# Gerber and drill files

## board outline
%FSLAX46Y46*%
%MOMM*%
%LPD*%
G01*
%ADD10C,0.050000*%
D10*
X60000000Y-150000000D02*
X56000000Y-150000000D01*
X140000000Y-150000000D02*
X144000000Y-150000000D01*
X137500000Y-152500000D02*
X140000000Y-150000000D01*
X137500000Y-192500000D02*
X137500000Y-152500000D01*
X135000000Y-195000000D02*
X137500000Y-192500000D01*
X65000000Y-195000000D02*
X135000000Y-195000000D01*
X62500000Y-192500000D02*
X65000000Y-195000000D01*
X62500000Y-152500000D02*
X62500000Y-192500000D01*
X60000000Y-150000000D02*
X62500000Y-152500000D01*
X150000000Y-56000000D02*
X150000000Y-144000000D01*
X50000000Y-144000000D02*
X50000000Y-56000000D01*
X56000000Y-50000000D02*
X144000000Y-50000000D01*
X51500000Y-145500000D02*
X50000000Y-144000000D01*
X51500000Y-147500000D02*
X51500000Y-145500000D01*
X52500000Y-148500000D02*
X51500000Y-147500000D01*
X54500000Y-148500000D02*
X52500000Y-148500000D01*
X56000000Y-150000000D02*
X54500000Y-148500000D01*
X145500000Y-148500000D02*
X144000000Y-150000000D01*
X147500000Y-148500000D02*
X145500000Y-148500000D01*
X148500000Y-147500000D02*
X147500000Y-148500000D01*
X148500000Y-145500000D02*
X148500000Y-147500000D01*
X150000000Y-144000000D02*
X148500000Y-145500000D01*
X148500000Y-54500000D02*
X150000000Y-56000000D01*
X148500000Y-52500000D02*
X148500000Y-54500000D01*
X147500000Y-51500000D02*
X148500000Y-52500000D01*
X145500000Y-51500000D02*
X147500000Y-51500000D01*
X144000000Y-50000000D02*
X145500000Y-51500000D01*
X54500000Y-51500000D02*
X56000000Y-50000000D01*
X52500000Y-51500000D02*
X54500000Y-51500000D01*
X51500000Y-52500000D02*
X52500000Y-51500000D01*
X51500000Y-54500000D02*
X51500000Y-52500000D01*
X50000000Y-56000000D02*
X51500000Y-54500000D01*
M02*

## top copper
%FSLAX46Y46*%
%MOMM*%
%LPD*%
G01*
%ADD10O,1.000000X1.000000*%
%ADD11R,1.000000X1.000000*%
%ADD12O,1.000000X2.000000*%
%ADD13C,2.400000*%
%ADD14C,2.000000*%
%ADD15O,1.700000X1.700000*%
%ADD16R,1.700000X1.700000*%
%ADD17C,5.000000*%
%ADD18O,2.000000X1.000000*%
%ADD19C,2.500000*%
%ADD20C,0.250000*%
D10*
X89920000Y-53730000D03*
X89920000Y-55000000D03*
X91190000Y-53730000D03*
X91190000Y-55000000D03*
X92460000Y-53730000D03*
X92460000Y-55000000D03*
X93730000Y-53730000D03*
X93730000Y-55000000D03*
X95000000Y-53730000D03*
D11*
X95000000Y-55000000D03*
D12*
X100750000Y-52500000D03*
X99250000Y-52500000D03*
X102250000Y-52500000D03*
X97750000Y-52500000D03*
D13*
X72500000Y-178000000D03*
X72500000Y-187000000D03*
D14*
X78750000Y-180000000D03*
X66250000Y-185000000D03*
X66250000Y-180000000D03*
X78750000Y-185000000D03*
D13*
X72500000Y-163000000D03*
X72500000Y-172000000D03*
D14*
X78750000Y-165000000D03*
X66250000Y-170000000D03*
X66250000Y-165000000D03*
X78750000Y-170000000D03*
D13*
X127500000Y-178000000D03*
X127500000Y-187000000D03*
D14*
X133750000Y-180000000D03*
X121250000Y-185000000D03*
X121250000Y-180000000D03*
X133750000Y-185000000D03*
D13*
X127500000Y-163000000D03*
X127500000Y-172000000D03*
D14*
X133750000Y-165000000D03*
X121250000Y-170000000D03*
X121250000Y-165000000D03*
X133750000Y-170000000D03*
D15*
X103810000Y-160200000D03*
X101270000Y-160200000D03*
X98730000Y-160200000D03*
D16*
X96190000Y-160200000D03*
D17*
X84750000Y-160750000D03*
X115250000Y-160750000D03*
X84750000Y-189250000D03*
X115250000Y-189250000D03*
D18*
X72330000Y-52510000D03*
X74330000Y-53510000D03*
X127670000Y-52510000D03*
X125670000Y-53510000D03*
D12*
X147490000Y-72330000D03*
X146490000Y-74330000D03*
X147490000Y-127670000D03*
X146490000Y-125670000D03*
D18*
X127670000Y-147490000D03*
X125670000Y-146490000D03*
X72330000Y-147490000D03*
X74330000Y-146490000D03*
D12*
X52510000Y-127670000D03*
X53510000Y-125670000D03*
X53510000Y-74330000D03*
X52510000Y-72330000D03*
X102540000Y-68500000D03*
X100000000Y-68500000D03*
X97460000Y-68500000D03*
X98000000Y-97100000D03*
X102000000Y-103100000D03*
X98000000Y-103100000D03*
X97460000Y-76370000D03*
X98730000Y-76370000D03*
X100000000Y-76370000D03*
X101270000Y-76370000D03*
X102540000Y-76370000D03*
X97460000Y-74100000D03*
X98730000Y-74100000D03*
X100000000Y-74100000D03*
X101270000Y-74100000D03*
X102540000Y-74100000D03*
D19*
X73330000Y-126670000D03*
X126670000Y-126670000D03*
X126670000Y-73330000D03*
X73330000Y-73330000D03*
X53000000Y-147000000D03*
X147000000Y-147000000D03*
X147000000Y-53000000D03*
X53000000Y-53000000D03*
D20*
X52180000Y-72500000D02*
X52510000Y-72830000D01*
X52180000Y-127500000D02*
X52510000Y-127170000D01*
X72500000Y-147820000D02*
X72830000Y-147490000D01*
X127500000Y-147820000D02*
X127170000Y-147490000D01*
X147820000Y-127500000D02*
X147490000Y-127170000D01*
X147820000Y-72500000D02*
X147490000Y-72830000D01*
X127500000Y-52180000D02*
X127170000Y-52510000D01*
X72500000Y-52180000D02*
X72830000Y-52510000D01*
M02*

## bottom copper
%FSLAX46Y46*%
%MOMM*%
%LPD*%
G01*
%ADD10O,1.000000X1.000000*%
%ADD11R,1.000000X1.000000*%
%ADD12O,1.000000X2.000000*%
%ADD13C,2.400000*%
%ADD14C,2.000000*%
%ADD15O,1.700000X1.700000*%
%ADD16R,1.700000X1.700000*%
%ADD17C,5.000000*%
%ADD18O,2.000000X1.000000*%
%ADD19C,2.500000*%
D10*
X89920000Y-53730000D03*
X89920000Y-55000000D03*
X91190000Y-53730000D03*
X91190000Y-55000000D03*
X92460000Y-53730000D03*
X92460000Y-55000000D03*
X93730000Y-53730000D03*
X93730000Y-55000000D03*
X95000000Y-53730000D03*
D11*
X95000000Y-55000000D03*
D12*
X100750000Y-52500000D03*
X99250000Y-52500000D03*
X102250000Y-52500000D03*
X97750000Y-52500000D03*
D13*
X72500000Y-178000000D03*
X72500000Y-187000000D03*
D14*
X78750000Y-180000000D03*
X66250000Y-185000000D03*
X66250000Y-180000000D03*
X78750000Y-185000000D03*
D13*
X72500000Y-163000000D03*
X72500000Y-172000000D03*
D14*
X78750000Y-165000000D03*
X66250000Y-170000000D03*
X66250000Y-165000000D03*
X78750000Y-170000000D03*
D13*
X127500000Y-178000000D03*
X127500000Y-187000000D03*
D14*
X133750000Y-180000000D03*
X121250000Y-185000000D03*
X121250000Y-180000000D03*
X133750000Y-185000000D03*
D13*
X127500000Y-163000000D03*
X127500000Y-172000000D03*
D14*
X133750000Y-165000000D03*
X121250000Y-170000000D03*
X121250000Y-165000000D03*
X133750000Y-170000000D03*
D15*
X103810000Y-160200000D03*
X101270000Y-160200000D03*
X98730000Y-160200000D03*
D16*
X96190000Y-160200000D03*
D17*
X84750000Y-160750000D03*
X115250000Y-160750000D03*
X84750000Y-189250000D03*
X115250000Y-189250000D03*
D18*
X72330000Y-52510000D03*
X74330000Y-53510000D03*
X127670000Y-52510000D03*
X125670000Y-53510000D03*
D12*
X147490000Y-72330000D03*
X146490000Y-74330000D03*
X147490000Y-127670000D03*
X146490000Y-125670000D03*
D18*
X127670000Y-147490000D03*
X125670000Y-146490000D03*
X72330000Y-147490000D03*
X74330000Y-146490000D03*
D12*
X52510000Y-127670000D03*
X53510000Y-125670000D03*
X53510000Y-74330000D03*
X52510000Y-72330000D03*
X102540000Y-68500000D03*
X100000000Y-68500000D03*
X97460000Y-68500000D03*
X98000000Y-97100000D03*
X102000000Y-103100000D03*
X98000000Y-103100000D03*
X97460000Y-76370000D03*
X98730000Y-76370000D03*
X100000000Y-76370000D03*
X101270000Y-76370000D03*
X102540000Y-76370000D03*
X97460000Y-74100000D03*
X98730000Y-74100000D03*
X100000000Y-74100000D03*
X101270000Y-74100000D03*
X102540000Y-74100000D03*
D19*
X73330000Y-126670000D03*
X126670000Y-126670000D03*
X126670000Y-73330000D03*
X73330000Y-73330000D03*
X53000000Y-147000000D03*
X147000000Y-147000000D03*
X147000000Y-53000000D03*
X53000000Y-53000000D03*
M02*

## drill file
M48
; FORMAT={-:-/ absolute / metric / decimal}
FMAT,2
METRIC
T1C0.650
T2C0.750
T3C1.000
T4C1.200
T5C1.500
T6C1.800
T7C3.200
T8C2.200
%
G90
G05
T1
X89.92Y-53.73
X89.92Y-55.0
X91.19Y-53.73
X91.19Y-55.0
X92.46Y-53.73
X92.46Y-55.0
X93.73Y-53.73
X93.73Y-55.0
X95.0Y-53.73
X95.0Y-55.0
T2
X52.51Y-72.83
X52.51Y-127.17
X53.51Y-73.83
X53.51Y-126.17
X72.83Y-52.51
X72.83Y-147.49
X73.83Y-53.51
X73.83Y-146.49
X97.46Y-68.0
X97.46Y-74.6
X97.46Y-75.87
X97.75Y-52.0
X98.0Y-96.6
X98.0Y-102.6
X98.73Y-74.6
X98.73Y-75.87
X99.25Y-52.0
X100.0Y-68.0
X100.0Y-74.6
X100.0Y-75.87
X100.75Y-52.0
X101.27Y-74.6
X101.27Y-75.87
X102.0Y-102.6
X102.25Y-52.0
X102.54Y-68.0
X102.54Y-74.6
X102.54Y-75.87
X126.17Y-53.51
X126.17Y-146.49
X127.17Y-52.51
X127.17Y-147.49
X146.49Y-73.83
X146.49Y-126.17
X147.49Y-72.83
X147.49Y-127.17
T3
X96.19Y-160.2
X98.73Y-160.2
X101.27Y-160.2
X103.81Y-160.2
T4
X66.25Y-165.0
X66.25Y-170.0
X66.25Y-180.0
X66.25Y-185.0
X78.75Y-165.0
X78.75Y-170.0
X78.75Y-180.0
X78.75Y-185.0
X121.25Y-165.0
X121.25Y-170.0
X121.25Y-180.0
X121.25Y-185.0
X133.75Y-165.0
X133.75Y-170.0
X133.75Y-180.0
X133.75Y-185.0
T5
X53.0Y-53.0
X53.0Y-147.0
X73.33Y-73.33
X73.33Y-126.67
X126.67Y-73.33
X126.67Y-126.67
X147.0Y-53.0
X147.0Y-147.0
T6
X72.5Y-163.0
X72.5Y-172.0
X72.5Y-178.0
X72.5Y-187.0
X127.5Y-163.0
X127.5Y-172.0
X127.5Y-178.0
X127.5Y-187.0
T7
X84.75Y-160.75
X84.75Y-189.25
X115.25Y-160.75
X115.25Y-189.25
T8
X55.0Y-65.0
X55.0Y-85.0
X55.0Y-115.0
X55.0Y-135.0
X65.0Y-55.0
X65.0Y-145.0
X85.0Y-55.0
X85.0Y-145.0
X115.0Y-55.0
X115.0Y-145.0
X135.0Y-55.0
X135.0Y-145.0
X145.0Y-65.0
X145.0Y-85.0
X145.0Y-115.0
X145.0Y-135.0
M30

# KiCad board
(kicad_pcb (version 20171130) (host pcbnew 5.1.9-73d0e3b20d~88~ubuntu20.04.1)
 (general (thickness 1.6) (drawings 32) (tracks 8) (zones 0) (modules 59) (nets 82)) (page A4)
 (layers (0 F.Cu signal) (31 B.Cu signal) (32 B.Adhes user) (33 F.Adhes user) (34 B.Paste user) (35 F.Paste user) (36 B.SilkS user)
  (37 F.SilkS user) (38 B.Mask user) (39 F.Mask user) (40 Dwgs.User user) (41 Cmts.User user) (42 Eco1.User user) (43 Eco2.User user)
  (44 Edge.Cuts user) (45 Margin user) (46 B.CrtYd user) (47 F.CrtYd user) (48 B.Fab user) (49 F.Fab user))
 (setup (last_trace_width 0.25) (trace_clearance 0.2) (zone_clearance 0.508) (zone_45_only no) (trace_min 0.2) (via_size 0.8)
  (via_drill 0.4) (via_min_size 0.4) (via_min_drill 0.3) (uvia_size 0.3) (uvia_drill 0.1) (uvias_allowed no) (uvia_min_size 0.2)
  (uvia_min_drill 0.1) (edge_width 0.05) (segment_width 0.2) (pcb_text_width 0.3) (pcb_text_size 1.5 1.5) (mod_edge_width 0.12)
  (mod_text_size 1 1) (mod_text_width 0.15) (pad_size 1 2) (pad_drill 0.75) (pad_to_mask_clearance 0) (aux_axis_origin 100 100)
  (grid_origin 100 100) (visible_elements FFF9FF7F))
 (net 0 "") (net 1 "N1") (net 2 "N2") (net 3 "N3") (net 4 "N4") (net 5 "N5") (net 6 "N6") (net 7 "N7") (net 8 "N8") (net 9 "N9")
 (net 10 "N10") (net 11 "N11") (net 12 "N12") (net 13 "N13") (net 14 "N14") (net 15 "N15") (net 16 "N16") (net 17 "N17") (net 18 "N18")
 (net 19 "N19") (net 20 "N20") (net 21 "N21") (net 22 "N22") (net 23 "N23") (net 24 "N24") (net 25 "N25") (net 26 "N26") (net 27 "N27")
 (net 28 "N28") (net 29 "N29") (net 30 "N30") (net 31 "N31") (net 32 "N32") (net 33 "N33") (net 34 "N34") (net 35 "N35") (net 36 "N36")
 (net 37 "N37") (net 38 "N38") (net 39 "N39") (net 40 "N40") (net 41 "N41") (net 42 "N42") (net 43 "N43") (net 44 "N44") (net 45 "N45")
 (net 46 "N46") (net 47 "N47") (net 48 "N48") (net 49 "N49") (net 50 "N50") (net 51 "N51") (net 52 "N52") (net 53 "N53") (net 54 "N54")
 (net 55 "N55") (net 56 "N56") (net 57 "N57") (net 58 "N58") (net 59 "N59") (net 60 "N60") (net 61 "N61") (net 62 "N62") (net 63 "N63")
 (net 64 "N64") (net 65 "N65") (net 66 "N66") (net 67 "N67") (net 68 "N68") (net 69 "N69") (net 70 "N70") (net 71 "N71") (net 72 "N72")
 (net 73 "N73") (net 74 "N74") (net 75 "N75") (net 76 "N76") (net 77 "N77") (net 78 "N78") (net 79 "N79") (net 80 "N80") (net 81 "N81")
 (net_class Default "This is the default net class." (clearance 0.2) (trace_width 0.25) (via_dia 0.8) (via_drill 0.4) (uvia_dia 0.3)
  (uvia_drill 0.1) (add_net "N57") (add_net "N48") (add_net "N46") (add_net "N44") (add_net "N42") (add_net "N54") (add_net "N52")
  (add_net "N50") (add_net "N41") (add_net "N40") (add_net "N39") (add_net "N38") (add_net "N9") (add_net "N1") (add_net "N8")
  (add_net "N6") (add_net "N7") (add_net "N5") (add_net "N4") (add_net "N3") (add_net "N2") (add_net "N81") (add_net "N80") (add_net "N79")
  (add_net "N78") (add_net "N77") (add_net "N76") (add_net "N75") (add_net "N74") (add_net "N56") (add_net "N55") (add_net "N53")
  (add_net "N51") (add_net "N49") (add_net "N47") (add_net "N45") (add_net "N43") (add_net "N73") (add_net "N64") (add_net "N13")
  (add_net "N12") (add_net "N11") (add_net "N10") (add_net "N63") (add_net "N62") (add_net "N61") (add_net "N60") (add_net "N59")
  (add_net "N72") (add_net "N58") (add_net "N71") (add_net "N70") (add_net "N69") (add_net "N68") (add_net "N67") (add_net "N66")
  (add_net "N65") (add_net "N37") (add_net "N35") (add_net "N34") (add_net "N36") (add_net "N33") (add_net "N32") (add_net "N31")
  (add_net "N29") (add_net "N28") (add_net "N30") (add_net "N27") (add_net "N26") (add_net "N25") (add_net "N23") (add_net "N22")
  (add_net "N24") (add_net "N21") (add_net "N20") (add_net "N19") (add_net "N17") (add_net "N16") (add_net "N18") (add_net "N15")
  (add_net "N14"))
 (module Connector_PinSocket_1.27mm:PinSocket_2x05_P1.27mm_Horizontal (layer F.Cu) (at 95 55 270)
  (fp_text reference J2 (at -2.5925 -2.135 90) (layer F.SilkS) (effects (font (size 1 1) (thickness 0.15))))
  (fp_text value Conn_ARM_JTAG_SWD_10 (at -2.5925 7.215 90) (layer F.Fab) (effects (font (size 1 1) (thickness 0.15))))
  (pad 10 thru_hole oval (at -1.27 5.08 270) (size 1 1) (drill 0.65) (layers *.Cu *.Mask) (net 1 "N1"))
  (pad 9 thru_hole oval (at 0 5.08 270) (size 1 1) (drill 0.65) (layers *.Cu *.Mask) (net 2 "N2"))
  (pad 8 thru_hole oval (at -1.27 3.81 270) (size 1 1) (drill 0.65) (layers *.Cu *.Mask) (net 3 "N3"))
  (pad 7 thru_hole oval (at 0 3.81 270) (size 1 1) (drill 0.65) (layers *.Cu *.Mask) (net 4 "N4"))
  (pad 6 thru_hole oval (at -1.27 2.54 270) (size 1 1) (drill 0.65) (layers *.Cu *.Mask) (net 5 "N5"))
  (pad 5 thru_hole oval (at 0 2.54 270) (size 1 1) (drill 0.65) (layers *.Cu *.Mask) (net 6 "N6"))
  (pad 4 thru_hole oval (at -1.27 1.27 270) (size 1 1) (drill 0.65) (layers *.Cu *.Mask) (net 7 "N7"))
  (pad 3 thru_hole oval (at 0 1.27 270) (size 1 1) (drill 0.65) (layers *.Cu *.Mask) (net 6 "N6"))
  (pad 2 thru_hole oval (at -1.27 0 270) (size 1 1) (drill 0.65) (layers *.Cu *.Mask) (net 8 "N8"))
  (pad 1 thru_hole rect (at 0 0 270) (size 1 1) (drill 0.65) (layers *.Cu *.Mask) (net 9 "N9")))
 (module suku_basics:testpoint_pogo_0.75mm (layer F.Cu) (at 100.75 52)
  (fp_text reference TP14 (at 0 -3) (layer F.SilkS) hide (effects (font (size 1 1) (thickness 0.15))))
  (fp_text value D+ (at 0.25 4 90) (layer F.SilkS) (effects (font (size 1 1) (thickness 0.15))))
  (pad 1 thru_hole oval (at 0 0) (size 1 2) (drill 0.75 (offset 0 0.5)) (layers *.Cu *.Mask) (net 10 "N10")))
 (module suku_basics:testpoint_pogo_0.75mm (layer F.Cu) (at 99.25 52)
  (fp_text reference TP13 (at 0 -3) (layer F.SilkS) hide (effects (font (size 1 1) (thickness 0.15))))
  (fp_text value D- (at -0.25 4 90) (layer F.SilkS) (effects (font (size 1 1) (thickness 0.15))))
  (pad 1 thru_hole oval (at 0 0) (size 1 2) (drill 0.75 (offset 0 0.5)) (layers *.Cu *.Mask) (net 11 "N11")))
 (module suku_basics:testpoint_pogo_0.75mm (layer F.Cu) (at 102.25 52)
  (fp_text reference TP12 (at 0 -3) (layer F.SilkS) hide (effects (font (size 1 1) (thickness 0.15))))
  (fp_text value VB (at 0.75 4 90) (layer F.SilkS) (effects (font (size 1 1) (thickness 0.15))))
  (pad 1 thru_hole oval (at 0 0) (size 1 2) (drill 0.75 (offset 0 0.5)) (layers *.Cu *.Mask) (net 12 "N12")))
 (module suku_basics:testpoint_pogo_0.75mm (layer F.Cu) (at 97.75 52)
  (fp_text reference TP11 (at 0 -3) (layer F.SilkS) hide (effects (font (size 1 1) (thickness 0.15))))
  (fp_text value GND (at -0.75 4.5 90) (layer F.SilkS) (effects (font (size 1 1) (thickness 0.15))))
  (pad 1 thru_hole oval (at 0 0) (size 1 2) (drill 0.75 (offset 0 0.5)) (layers *.Cu *.Mask) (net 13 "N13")))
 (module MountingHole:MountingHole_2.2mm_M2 (layer F.Cu) (at 145 135)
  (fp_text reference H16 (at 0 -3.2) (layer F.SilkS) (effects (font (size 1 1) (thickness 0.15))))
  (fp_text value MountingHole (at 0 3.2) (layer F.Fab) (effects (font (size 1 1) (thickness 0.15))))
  (pad 1 np_thru_hole circle (at 0 0) (size 2.2 2.2) (drill 2.2) (layers *.Cu *.Mask)))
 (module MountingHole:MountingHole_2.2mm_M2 (layer F.Cu) (at 65 145)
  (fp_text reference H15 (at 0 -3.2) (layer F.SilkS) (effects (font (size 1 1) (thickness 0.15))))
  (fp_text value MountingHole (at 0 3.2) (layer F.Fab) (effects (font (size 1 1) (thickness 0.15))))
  (pad 1 np_thru_hole circle (at 0 0) (size 2.2 2.2) (drill 2.2) (layers *.Cu *.Mask)))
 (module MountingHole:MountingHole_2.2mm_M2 (layer F.Cu) (at 135 145)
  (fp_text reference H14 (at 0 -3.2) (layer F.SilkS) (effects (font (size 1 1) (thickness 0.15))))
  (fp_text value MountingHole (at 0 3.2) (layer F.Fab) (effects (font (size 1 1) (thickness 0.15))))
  (pad 1 np_thru_hole circle (at 0 0) (size 2.2 2.2) (drill 2.2) (layers *.Cu *.Mask)))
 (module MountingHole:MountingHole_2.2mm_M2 (layer F.Cu) (at 55 135)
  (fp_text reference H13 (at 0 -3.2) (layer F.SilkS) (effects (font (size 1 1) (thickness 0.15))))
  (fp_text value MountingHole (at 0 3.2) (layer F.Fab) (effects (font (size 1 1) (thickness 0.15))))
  (pad 1 np_thru_hole circle (at 0 0) (size 2.2 2.2) (drill 2.2) (layers *.Cu *.Mask)))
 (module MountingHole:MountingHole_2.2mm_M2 (layer F.Cu) (at 135 55)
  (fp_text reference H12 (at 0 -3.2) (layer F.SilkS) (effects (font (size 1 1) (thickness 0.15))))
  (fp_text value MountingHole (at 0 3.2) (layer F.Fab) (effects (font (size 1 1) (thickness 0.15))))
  (pad 1 np_thru_hole circle (at 0 0) (size 2.2 2.2) (drill 2.2) (layers *.Cu *.Mask)))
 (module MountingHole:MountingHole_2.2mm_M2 (layer F.Cu) (at 65 55)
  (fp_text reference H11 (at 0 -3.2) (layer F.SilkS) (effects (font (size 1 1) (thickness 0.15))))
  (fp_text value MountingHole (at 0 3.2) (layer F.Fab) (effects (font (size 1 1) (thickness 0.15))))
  (pad 1 np_thru_hole circle (at 0 0) (size 2.2 2.2) (drill 2.2) (layers *.Cu *.Mask)))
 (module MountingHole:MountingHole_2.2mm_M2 (layer F.Cu) (at 145 65)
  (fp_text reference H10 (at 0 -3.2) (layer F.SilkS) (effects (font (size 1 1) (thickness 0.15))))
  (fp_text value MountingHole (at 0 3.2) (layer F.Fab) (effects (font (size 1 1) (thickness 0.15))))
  (pad 1 np_thru_hole circle (at 0 0) (size 2.2 2.2) (drill 2.2) (layers *.Cu *.Mask)))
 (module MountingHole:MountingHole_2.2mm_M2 (layer F.Cu) (at 55 65)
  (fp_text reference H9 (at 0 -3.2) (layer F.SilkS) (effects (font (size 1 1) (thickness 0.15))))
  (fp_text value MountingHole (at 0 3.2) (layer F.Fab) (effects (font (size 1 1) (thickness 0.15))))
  (pad 1 np_thru_hole circle (at 0 0) (size 2.2 2.2) (drill 2.2) (layers *.Cu *.Mask)))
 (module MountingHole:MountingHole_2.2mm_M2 (layer F.Cu) (at 55 115)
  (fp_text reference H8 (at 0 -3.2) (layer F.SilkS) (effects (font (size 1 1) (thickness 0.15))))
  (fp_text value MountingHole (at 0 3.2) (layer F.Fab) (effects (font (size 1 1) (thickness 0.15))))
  (pad 1 np_thru_hole circle (at 0 0) (size 2.2 2.2) (drill 2.2) (layers *.Cu *.Mask)))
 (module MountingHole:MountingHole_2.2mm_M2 (layer F.Cu) (at 55 85)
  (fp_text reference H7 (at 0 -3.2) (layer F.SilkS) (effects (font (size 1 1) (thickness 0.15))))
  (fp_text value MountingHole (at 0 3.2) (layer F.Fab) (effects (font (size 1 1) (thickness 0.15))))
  (pad 1 np_thru_hole circle (at 0 0) (size 2.2 2.2) (drill 2.2) (layers *.Cu *.Mask)))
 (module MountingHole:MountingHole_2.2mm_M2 (layer F.Cu) (at 145 115)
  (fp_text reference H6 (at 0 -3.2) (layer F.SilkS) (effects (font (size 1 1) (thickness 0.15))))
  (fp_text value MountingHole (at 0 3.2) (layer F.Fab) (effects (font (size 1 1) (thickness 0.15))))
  (pad 1 np_thru_hole circle (at 0 0) (size 2.2 2.2) (drill 2.2) (layers *.Cu *.Mask)))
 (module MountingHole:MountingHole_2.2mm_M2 (layer F.Cu) (at 145 85)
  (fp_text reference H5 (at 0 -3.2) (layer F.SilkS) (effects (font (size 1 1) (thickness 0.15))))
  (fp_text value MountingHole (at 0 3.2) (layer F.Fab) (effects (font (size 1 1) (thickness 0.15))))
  (pad 1 np_thru_hole circle (at 0 0) (size 2.2 2.2) (drill 2.2) (layers *.Cu *.Mask)))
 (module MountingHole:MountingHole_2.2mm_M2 (layer F.Cu) (at 85 145)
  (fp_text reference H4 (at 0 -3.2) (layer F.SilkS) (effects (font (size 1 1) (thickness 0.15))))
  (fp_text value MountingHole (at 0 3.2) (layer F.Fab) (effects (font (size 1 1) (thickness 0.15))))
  (pad 1 np_thru_hole circle (at 0 0) (size 2.2 2.2) (drill 2.2) (layers *.Cu *.Mask)))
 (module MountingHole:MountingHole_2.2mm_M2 (layer F.Cu) (at 115 55)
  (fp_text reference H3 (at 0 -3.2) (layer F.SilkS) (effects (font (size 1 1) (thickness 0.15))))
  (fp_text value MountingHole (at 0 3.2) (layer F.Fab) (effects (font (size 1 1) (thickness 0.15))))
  (pad 1 np_thru_hole circle (at 0 0) (size 2.2 2.2) (drill 2.2) (layers *.Cu *.Mask)))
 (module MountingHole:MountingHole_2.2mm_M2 (layer F.Cu) (at 115 145)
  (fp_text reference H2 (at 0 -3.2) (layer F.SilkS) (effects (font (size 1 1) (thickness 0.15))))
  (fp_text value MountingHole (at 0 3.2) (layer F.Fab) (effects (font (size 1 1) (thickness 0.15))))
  (pad 1 np_thru_hole circle (at 0 0) (size 2.2 2.2) (drill 2.2) (layers *.Cu *.Mask)))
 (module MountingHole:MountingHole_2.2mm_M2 (layer F.Cu) (at 85 55)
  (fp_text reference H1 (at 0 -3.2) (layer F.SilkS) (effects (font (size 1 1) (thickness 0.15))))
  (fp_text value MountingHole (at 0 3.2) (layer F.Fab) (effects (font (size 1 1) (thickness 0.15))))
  (pad 1 np_thru_hole circle (at 0 0) (size 2.2 2.2) (drill 2.2) (layers *.Cu *.Mask)))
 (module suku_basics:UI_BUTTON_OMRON (layer F.Cu) (at 72.5 182.5)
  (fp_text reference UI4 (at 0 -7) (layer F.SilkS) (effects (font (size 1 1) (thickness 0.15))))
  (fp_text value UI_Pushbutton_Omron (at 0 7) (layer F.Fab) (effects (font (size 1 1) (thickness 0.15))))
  (pad 6 thru_hole circle (at 0 -4.5 270) (size 2.4 2.4) (drill 1.8) (layers *.Cu *.Mask) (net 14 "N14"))
  (pad 5 thru_hole circle (at 0 4.5 270) (size 2.4 2.4) (drill 1.8) (layers *.Cu *.Mask) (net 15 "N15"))
  (pad 3 thru_hole circle (at 6.25 -2.5 180) (size 2 2) (drill 1.2) (layers *.Cu *.Mask) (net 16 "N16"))
  (pad 2 thru_hole circle (at -6.25 2.5 180) (size 2 2) (drill 1.2) (layers *.Cu *.Mask) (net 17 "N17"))
  (pad 4 thru_hole circle (at -6.25 -2.5 270) (size 2 2) (drill 1.2) (layers *.Cu *.Mask) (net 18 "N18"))
  (pad 1 thru_hole circle (at 6.25 2.5) (size 2 2) (drill 1.2) (layers *.Cu *.Mask) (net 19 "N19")))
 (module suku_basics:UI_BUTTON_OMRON (layer F.Cu) (at 72.5 167.5)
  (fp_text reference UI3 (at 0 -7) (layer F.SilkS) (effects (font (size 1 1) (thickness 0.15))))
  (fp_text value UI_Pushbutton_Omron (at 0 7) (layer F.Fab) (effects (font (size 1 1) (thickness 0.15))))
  (pad 6 thru_hole circle (at 0 -4.5 270) (size 2.4 2.4) (drill 1.8) (layers *.Cu *.Mask) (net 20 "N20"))
  (pad 5 thru_hole circle (at 0 4.5 270) (size 2.4 2.4) (drill 1.8) (layers *.Cu *.Mask) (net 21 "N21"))
  (pad 3 thru_hole circle (at 6.25 -2.5 180) (size 2 2) (drill 1.2) (layers *.Cu *.Mask) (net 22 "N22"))
  (pad 2 thru_hole circle (at -6.25 2.5 180) (size 2 2) (drill 1.2) (layers *.Cu *.Mask) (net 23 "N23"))
  (pad 4 thru_hole circle (at -6.25 -2.5 270) (size 2 2) (drill 1.2) (layers *.Cu *.Mask) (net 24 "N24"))
  (pad 1 thru_hole circle (at 6.25 2.5) (size 2 2) (drill 1.2) (layers *.Cu *.Mask) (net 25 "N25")))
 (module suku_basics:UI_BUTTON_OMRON (layer F.Cu) (at 127.5 182.5)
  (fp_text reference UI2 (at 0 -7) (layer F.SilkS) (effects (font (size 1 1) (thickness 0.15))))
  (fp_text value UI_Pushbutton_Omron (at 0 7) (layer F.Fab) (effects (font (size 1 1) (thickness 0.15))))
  (pad 6 thru_hole circle (at 0 -4.5 270) (size 2.4 2.4) (drill 1.8) (layers *.Cu *.Mask) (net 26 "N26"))
  (pad 5 thru_hole circle (at 0 4.5 270) (size 2.4 2.4) (drill 1.8) (layers *.Cu *.Mask) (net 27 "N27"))
  (pad 3 thru_hole circle (at 6.25 -2.5 180) (size 2 2) (drill 1.2) (layers *.Cu *.Mask) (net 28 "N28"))
  (pad 2 thru_hole circle (at -6.25 2.5 180) (size 2 2) (drill 1.2) (layers *.Cu *.Mask) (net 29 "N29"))
  (pad 4 thru_hole circle (at -6.25 -2.5 270) (size 2 2) (drill 1.2) (layers *.Cu *.Mask) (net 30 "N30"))
  (pad 1 thru_hole circle (at 6.25 2.5) (size 2 2) (drill 1.2) (layers *.Cu *.Mask) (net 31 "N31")))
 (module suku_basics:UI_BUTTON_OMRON (layer F.Cu) (at 127.5 167.5)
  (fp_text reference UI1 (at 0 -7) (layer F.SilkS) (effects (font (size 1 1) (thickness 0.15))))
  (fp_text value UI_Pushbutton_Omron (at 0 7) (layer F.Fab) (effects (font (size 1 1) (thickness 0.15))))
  (pad 6 thru_hole circle (at 0 -4.5 270) (size 2.4 2.4) (drill 1.8) (layers *.Cu *.Mask) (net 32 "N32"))
  (pad 5 thru_hole circle (at 0 4.5 270) (size 2.4 2.4) (drill 1.8) (layers *.Cu *.Mask) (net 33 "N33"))
  (pad 3 thru_hole circle (at 6.25 -2.5 180) (size 2 2) (drill 1.2) (layers *.Cu *.Mask) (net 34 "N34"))
  (pad 2 thru_hole circle (at -6.25 2.5 180) (size 2 2) (drill 1.2) (layers *.Cu *.Mask) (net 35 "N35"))
  (pad 4 thru_hole circle (at -6.25 -2.5 270) (size 2 2) (drill 1.2) (layers *.Cu *.Mask) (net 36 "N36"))
  (pad 1 thru_hole circle (at 6.25 2.5) (size 2 2) (drill 1.2) (layers *.Cu *.Mask) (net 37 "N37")))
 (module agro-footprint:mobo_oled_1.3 (layer F.Cu) (at 100 175)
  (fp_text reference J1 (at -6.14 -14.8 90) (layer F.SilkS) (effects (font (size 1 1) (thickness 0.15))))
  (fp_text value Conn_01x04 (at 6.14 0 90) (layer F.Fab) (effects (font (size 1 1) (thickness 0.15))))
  (pad 4 thru_hole oval (at 3.81 -14.8 90) (size 1.7 1.7) (drill 1) (layers *.Cu *.Mask) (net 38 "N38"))
  (pad 3 thru_hole oval (at 1.27 -14.8 90) (size 1.7 1.7) (drill 1) (layers *.Cu *.Mask) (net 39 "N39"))
  (pad 2 thru_hole oval (at -1.27 -14.8 90) (size 1.7 1.7) (drill 1) (layers *.Cu *.Mask) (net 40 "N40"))
  (pad 1 thru_hole rect (at -3.81 -14.8 90) (size 1.7 1.7) (drill 1) (layers *.Cu *.Mask) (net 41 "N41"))
  (pad "" thru_hole circle (at -15.25 -14.25) (size 5 5) (drill 3.2) (layers *.Cu *.Mask))
  (pad "" thru_hole circle (at 15.25 -14.25) (size 5 5) (drill 3.2) (layers *.Cu *.Mask))
  (pad "" thru_hole circle (at -15.25 14.25) (size 5 5) (drill 3.2) (layers *.Cu *.Mask))
  (pad "" thru_hole circle (at 15.25 14.25) (size 5 5) (drill 3.2) (layers *.Cu *.Mask)))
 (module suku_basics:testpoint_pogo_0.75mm (layer F.Cu) (at 72.83 52.51 270)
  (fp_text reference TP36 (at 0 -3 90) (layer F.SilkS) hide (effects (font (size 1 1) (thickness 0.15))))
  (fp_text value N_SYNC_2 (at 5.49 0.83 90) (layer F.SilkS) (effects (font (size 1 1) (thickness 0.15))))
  (pad 1 thru_hole oval (at 0 0 270) (size 1 2) (drill 0.75 (offset 0 0.5)) (layers *.Cu *.Mask) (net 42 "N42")))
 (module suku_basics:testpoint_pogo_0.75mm (layer F.Cu) (at 73.83 53.51 90)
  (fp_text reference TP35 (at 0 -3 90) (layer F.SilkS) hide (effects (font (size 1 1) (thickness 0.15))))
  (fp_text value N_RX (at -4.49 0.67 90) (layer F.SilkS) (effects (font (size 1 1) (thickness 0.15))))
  (pad 1 thru_hole oval (at 0 0 90) (size 1 2) (drill 0.75 (offset 0 0.5)) (layers *.Cu *.Mask) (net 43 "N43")))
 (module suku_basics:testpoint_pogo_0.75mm (layer F.Cu) (at 127.17 52.51 90)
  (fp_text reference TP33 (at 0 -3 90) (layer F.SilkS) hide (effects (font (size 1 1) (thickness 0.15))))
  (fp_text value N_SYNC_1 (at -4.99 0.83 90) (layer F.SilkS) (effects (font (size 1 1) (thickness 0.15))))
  (pad 1 thru_hole oval (at 0 0 90) (size 1 2) (drill 0.75 (offset 0 0.5)) (layers *.Cu *.Mask) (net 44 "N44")))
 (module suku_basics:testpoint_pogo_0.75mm (layer F.Cu) (at 126.17 53.51 270)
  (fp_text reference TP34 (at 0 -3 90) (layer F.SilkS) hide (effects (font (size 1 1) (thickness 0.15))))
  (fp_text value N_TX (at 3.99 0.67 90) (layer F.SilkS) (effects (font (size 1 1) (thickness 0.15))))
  (pad 1 thru_hole oval (at 0 0 270) (size 1 2) (drill 0.75 (offset 0 0.5)) (layers *.Cu *.Mask) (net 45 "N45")))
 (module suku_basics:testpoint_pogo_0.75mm (layer F.Cu) (at 147.49 72.83 180)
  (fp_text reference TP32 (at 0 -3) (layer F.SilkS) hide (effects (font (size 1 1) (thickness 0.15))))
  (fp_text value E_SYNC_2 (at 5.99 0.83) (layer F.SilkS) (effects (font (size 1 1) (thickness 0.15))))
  (pad 1 thru_hole oval (at 0 0 180) (size 1 2) (drill 0.75 (offset 0 0.5)) (layers *.Cu *.Mask) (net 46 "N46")))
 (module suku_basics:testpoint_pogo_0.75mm (layer F.Cu) (at 146.49 73.83)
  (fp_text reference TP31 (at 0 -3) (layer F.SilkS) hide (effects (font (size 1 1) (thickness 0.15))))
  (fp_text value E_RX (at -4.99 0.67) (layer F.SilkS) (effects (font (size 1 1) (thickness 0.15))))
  (pad 1 thru_hole oval (at 0 0) (size 1 2) (drill 0.75 (offset 0 0.5)) (layers *.Cu *.Mask) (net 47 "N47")))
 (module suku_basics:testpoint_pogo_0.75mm (layer F.Cu) (at 147.49 127.17)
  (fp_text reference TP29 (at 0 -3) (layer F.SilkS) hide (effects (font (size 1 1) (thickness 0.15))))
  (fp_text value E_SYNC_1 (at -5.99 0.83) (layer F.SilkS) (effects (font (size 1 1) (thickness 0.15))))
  (pad 1 thru_hole oval (at 0 0) (size 1 2) (drill 0.75 (offset 0 0.5)) (layers *.Cu *.Mask) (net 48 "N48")))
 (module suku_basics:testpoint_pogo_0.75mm (layer F.Cu) (at 146.49 126.17 180)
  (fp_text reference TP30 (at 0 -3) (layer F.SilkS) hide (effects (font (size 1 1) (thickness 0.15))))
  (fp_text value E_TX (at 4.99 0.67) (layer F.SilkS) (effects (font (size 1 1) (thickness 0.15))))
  (pad 1 thru_hole oval (at 0 0 180) (size 1 2) (drill 0.75 (offset 0 0.5)) (layers *.Cu *.Mask) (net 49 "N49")))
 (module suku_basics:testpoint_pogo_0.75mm (layer F.Cu) (at 127.17 147.49 90)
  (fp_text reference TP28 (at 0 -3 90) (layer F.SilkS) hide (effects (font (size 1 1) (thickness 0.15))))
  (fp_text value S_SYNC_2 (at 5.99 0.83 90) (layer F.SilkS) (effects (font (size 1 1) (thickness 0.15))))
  (pad 1 thru_hole oval (at 0 0 90) (size 1 2) (drill 0.75 (offset 0 0.5)) (layers *.Cu *.Mask) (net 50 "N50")))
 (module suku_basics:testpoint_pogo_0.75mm (layer F.Cu) (at 126.17 146.49 270)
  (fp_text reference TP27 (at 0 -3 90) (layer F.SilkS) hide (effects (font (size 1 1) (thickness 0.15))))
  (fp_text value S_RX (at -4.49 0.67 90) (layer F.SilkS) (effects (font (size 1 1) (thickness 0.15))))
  (pad 1 thru_hole oval (at 0 0 270) (size 1 2) (drill 0.75 (offset 0 0.5)) (layers *.Cu *.Mask) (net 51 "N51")))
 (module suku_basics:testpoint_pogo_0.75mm (layer F.Cu) (at 72.83 147.49 270)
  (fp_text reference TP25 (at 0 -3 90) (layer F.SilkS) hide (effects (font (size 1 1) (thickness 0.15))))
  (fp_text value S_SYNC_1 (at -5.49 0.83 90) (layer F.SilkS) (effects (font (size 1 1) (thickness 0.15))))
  (pad 1 thru_hole oval (at 0 0 270) (size 1 2) (drill 0.75 (offset 0 0.5)) (layers *.Cu *.Mask) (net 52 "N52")))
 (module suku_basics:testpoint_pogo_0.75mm (layer F.Cu) (at 73.83 146.49 90)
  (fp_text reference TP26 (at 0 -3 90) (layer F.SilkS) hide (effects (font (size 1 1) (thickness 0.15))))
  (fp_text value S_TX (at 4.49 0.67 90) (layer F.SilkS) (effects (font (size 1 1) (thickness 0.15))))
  (pad 1 thru_hole oval (at 0 0 90) (size 1 2) (drill 0.75 (offset 0 0.5)) (layers *.Cu *.Mask) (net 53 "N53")))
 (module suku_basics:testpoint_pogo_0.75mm (layer F.Cu) (at 52.51 127.17)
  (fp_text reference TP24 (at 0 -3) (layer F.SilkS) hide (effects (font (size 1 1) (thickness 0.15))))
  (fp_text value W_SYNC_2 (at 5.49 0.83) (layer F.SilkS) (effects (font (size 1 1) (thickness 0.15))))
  (pad 1 thru_hole oval (at 0 0) (size 1 2) (drill 0.75 (offset 0 0.5)) (layers *.Cu *.Mask) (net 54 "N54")))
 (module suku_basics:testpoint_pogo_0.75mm (layer F.Cu) (at 53.51 126.17 180)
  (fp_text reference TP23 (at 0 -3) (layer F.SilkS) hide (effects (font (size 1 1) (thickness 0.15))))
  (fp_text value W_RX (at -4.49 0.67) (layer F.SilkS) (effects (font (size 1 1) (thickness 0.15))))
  (pad 1 thru_hole oval (at 0 0 180) (size 1 2) (drill 0.75 (offset 0 0.5)) (layers *.Cu *.Mask) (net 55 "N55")))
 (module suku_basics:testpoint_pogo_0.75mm (layer F.Cu) (at 53.51 73.83)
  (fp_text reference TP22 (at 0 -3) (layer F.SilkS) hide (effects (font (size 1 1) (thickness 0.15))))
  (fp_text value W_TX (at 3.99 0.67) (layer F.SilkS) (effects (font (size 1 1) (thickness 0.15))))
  (pad 1 thru_hole oval (at 0 0) (size 1 2) (drill 0.75 (offset 0 0.5)) (layers *.Cu *.Mask) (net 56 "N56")))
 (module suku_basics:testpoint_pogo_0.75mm (layer F.Cu) (at 52.51 72.83 180)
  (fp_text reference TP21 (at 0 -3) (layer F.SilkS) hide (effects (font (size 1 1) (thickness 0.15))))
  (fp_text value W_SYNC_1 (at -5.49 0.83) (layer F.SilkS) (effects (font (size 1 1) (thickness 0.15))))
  (pad 1 thru_hole oval (at 0 0 180) (size 1 2) (drill 0.75 (offset 0 0.5)) (layers *.Cu *.Mask) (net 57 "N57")))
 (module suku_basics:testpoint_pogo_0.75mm (layer F.Cu) (at 102.54 68)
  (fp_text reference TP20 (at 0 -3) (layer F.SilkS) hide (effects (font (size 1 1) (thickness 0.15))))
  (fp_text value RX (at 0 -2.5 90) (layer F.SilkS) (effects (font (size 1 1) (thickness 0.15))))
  (pad 1 thru_hole oval (at 0 0) (size 1 2) (drill 0.75 (offset 0 0.5)) (layers *.Cu *.Mask) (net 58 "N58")))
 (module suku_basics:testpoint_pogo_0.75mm (layer F.Cu) (at 100 68)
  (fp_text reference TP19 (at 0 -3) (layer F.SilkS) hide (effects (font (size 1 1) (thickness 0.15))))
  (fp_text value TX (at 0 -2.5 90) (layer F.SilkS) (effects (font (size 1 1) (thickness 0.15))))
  (pad 1 thru_hole oval (at 0 0) (size 1 2) (drill 0.75 (offset 0 0.5)) (layers *.Cu *.Mask) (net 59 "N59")))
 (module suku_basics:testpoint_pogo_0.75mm (layer F.Cu) (at 97.46 68)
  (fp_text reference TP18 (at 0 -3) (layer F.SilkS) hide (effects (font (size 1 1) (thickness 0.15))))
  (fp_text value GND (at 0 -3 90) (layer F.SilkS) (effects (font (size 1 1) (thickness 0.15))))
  (pad 1 thru_hole oval (at 0 0) (size 1 2) (drill 0.75 (offset 0 0.5)) (layers *.Cu *.Mask) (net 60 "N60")))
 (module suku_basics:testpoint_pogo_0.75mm (layer F.Cu) (at 98 96.6)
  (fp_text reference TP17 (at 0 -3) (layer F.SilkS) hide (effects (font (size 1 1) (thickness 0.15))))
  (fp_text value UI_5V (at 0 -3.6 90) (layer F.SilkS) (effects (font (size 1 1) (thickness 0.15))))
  (pad 1 thru_hole oval (at 0 0) (size 1 2) (drill 0.75 (offset 0 0.5)) (layers *.Cu *.Mask) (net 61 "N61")))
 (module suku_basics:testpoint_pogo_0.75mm (layer F.Cu) (at 102 102.6)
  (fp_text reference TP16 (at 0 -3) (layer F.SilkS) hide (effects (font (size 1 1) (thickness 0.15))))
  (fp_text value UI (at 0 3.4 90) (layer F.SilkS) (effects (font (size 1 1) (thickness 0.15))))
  (pad 1 thru_hole oval (at 0 0) (size 1 2) (drill 0.75 (offset 0 0.5)) (layers *.Cu *.Mask) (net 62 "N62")))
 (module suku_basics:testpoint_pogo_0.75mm (layer F.Cu) (at 98 102.6)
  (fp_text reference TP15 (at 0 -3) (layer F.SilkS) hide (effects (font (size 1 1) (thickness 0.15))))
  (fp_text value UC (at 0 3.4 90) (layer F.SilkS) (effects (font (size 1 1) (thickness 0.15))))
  (pad 1 thru_hole oval (at 0 0) (size 1 2) (drill 0.75 (offset 0 0.5)) (layers *.Cu *.Mask) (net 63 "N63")))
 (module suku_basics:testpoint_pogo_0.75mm (layer F.Cu) (at 97.46 75.87)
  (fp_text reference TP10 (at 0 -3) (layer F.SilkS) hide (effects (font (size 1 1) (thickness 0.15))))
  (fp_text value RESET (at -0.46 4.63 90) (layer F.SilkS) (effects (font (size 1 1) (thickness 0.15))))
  (pad 1 thru_hole oval (at 0 0) (size 1 2) (drill 0.75 (offset 0 0.5)) (layers *.Cu *.Mask) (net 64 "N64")))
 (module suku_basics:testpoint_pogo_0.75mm (layer F.Cu) (at 98.73 75.87)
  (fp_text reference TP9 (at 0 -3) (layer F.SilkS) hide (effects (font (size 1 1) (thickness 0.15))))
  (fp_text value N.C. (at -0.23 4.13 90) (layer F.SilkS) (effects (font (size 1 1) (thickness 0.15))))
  (pad 1 thru_hole oval (at 0 0) (size 1 2) (drill 0.75 (offset 0 0.5)) (layers *.Cu *.Mask) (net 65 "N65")))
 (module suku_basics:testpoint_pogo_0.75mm (layer F.Cu) (at 100 75.87)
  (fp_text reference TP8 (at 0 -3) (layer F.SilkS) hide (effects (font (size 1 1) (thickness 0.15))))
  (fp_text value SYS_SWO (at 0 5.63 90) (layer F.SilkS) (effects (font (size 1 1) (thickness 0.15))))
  (pad 1 thru_hole oval (at 0 0) (size 1 2) (drill 0.75 (offset 0 0.5)) (layers *.Cu *.Mask) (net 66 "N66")))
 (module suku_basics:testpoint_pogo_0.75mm (layer F.Cu) (at 101.27 75.87)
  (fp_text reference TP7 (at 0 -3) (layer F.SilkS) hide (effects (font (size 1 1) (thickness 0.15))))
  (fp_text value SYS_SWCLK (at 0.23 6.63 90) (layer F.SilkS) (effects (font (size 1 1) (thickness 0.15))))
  (pad 1 thru_hole oval (at 0 0) (size 1 2) (drill 0.75 (offset 0 0.5)) (layers *.Cu *.Mask) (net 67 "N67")))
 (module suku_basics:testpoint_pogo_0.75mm (layer F.Cu) (at 102.54 75.87)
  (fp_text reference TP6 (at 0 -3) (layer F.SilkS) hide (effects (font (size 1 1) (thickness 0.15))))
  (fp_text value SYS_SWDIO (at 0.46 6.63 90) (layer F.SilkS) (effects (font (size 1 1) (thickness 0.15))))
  (pad 1 thru_hole oval (at 0 0) (size 1 2) (drill 0.75 (offset 0 0.5)) (layers *.Cu *.Mask) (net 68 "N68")))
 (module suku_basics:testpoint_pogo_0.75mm (layer F.Cu) (at 97.46 74.6 180)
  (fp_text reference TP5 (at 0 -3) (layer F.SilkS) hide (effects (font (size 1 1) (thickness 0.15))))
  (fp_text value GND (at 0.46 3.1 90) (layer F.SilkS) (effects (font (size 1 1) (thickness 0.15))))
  (pad 1 thru_hole oval (at 0 0 180) (size 1 2) (drill 0.75 (offset 0 0.5)) (layers *.Cu *.Mask) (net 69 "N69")))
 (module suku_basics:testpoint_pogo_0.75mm (layer F.Cu) (at 98.73 74.6 180)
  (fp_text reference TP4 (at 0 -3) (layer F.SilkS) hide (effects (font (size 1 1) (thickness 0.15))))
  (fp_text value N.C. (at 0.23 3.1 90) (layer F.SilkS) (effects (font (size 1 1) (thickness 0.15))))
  (pad 1 thru_hole oval (at 0 0 180) (size 1 2) (drill 0.75 (offset 0 0.5)) (layers *.Cu *.Mask) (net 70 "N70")))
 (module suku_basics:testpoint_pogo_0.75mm (layer F.Cu) (at 100 74.6 180)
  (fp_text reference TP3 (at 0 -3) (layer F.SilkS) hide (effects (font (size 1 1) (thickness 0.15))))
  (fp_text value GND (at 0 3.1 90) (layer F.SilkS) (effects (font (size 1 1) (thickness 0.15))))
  (pad 1 thru_hole oval (at 0 0 180) (size 1 2) (drill 0.75 (offset 0 0.5)) (layers *.Cu *.Mask) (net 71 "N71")))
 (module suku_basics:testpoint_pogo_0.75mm (layer F.Cu) (at 101.27 74.6 180)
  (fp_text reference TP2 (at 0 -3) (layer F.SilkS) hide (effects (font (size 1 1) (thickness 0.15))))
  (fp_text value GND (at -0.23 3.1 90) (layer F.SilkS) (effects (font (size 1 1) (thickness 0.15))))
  (pad 1 thru_hole oval (at 0 0 180) (size 1 2) (drill 0.75 (offset 0 0.5)) (layers *.Cu *.Mask) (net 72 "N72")))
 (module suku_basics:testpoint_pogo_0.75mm (layer F.Cu) (at 102.54 74.6 180)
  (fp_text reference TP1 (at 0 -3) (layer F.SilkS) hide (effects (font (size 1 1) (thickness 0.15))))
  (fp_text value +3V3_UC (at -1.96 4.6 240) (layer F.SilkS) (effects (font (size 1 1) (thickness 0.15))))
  (pad 1 thru_hole oval (at 0 0 180) (size 1 2) (drill 0.75 (offset 0 0.5)) (layers *.Cu *.Mask) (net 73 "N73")))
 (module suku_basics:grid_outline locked (layer F.Cu) (at 100 100)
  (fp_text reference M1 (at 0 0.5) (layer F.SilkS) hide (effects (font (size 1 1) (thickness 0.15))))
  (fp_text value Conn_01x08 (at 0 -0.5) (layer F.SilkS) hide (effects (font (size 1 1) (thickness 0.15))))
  (pad 8 thru_hole circle (at -26.67 26.67) (size 2.5 2.5) (drill 1.5) (layers *.Cu *.Mask) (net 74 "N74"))
  (pad 7 thru_hole circle (at 26.67 26.67) (size 2.5 2.5) (drill 1.5) (layers *.Cu *.Mask) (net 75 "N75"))
  (pad 6 thru_hole circle (at 26.67 -26.67) (size 2.5 2.5) (drill 1.5) (layers *.Cu *.Mask) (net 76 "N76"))
  (pad 5 thru_hole circle (at -26.67 -26.67) (size 2.5 2.5) (drill 1.5) (layers *.Cu *.Mask) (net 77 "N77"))
  (pad 4 thru_hole circle (at -47 47) (size 2.5 2.5) (drill 1.5) (layers *.Cu *.Mask) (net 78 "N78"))
  (pad 3 thru_hole circle (at 47 47) (size 2.5 2.5) (drill 1.5) (layers *.Cu *.Mask) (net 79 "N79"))
  (pad 2 thru_hole circle (at 47 -47) (size 2.5 2.5) (drill 1.5) (layers *.Cu *.Mask) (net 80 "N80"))
  (pad 1 thru_hole circle (at -47 -47) (size 2.5 2.5) (drill 1.5) (layers *.Cu *.Mask) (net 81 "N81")))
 (gr_line (start 60 150) (end 56 150) (layer Edge.Cuts) (width 0.05))
 (gr_line (start 140 150) (end 144 150) (layer Edge.Cuts) (width 0.05))
 (gr_line (start 137.5 152.5) (end 140 150) (layer Edge.Cuts) (width 0.05))
 (gr_line (start 137.5 192.5) (end 137.5 152.5) (layer Edge.Cuts) (width 0.05))
 (gr_line (start 135 195) (end 137.5 192.5) (layer Edge.Cuts) (width 0.05))
 (gr_line (start 65 195) (end 135 195) (layer Edge.Cuts) (width 0.05))
 (gr_line (start 62.5 192.5) (end 65 195) (layer Edge.Cuts) (width 0.05))
 (gr_line (start 62.5 152.5) (end 62.5 192.5) (layer Edge.Cuts) (width 0.05))
 (gr_line (start 60 150) (end 62.5 152.5) (layer Edge.Cuts) (width 0.05))
 (gr_line (start 150 56) (end 150 144) (layer Edge.Cuts) (width 0.05))
 (gr_line (start 50 144) (end 50 56) (layer Edge.Cuts) (width 0.05))
 (gr_line (start 56 50) (end 144 50) (layer Edge.Cuts) (width 0.05))
 (gr_line (start 51.5 145.5) (end 50 144) (layer Edge.Cuts) (width 0.05))
 (gr_line (start 51.5 147.5) (end 51.5 145.5) (layer Edge.Cuts) (width 0.05))
 (gr_line (start 52.5 148.5) (end 51.5 147.5) (layer Edge.Cuts) (width 0.05))
 (gr_line (start 54.5 148.5) (end 52.5 148.5) (layer Edge.Cuts) (width 0.05))
 (gr_line (start 56 150) (end 54.5 148.5) (layer Edge.Cuts) (width 0.05))
 (gr_line (start 145.5 148.5) (end 144 150) (layer Edge.Cuts) (width 0.05))
 (gr_line (start 147.5 148.5) (end 145.5 148.5) (layer Edge.Cuts) (width 0.05))
 (gr_line (start 148.5 147.5) (end 147.5 148.5) (layer Edge.Cuts) (width 0.05))
 (gr_line (start 148.5 145.5) (end 148.5 147.5) (layer Edge.Cuts) (width 0.05))
 (gr_line (start 150 144) (end 148.5 145.5) (layer Edge.Cuts) (width 0.05))
 (gr_line (start 148.5 54.5) (end 150 56) (layer Edge.Cuts) (width 0.05))
 (gr_line (start 148.5 52.5) (end 148.5 54.5) (layer Edge.Cuts) (width 0.05))
 (gr_line (start 147.5 51.5) (end 148.5 52.5) (layer Edge.Cuts) (width 0.05))
 (gr_line (start 145.5 51.5) (end 147.5 51.5) (layer Edge.Cuts) (width 0.05))
 (gr_line (start 144 50) (end 145.5 51.5) (layer Edge.Cuts) (width 0.05))
 (gr_line (start 54.5 51.5) (end 56 50) (layer Edge.Cuts) (width 0.05))
 (gr_line (start 52.5 51.5) (end 54.5 51.5) (layer Edge.Cuts) (width 0.05))
 (gr_line (start 51.5 52.5) (end 52.5 51.5) (layer Edge.Cuts) (width 0.05))
 (gr_line (start 51.5 54.5) (end 51.5 52.5) (layer Edge.Cuts) (width 0.05))
 (gr_line (start 50 56) (end 51.5 54.5) (layer Edge.Cuts) (width 0.05))
 (segment (start 52.18 72.5) (end 52.51 72.83) (width 0.25) (layer F.Cu) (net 57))
 (segment (start 52.18 127.5) (end 52.51 127.17) (width 0.25) (layer F.Cu) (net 54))
 (segment (start 72.5 147.82) (end 72.83 147.49) (width 0.25) (layer F.Cu) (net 52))
 (segment (start 127.5 147.82) (end 127.17 147.49) (width 0.25) (layer F.Cu) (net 50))
 (segment (start 147.82 127.5) (end 147.49 127.17) (width 0.25) (layer F.Cu) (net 48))
 (segment (start 147.82 72.5) (end 147.49 72.83) (width 0.25) (layer F.Cu) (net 46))
 (segment (start 127.5 52.18) (end 127.17 52.51) (width 0.25) (layer F.Cu) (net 44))
 (segment (start 72.5 52.18) (end 72.83 52.51) (width 0.25) (layer F.Cu) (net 42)))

